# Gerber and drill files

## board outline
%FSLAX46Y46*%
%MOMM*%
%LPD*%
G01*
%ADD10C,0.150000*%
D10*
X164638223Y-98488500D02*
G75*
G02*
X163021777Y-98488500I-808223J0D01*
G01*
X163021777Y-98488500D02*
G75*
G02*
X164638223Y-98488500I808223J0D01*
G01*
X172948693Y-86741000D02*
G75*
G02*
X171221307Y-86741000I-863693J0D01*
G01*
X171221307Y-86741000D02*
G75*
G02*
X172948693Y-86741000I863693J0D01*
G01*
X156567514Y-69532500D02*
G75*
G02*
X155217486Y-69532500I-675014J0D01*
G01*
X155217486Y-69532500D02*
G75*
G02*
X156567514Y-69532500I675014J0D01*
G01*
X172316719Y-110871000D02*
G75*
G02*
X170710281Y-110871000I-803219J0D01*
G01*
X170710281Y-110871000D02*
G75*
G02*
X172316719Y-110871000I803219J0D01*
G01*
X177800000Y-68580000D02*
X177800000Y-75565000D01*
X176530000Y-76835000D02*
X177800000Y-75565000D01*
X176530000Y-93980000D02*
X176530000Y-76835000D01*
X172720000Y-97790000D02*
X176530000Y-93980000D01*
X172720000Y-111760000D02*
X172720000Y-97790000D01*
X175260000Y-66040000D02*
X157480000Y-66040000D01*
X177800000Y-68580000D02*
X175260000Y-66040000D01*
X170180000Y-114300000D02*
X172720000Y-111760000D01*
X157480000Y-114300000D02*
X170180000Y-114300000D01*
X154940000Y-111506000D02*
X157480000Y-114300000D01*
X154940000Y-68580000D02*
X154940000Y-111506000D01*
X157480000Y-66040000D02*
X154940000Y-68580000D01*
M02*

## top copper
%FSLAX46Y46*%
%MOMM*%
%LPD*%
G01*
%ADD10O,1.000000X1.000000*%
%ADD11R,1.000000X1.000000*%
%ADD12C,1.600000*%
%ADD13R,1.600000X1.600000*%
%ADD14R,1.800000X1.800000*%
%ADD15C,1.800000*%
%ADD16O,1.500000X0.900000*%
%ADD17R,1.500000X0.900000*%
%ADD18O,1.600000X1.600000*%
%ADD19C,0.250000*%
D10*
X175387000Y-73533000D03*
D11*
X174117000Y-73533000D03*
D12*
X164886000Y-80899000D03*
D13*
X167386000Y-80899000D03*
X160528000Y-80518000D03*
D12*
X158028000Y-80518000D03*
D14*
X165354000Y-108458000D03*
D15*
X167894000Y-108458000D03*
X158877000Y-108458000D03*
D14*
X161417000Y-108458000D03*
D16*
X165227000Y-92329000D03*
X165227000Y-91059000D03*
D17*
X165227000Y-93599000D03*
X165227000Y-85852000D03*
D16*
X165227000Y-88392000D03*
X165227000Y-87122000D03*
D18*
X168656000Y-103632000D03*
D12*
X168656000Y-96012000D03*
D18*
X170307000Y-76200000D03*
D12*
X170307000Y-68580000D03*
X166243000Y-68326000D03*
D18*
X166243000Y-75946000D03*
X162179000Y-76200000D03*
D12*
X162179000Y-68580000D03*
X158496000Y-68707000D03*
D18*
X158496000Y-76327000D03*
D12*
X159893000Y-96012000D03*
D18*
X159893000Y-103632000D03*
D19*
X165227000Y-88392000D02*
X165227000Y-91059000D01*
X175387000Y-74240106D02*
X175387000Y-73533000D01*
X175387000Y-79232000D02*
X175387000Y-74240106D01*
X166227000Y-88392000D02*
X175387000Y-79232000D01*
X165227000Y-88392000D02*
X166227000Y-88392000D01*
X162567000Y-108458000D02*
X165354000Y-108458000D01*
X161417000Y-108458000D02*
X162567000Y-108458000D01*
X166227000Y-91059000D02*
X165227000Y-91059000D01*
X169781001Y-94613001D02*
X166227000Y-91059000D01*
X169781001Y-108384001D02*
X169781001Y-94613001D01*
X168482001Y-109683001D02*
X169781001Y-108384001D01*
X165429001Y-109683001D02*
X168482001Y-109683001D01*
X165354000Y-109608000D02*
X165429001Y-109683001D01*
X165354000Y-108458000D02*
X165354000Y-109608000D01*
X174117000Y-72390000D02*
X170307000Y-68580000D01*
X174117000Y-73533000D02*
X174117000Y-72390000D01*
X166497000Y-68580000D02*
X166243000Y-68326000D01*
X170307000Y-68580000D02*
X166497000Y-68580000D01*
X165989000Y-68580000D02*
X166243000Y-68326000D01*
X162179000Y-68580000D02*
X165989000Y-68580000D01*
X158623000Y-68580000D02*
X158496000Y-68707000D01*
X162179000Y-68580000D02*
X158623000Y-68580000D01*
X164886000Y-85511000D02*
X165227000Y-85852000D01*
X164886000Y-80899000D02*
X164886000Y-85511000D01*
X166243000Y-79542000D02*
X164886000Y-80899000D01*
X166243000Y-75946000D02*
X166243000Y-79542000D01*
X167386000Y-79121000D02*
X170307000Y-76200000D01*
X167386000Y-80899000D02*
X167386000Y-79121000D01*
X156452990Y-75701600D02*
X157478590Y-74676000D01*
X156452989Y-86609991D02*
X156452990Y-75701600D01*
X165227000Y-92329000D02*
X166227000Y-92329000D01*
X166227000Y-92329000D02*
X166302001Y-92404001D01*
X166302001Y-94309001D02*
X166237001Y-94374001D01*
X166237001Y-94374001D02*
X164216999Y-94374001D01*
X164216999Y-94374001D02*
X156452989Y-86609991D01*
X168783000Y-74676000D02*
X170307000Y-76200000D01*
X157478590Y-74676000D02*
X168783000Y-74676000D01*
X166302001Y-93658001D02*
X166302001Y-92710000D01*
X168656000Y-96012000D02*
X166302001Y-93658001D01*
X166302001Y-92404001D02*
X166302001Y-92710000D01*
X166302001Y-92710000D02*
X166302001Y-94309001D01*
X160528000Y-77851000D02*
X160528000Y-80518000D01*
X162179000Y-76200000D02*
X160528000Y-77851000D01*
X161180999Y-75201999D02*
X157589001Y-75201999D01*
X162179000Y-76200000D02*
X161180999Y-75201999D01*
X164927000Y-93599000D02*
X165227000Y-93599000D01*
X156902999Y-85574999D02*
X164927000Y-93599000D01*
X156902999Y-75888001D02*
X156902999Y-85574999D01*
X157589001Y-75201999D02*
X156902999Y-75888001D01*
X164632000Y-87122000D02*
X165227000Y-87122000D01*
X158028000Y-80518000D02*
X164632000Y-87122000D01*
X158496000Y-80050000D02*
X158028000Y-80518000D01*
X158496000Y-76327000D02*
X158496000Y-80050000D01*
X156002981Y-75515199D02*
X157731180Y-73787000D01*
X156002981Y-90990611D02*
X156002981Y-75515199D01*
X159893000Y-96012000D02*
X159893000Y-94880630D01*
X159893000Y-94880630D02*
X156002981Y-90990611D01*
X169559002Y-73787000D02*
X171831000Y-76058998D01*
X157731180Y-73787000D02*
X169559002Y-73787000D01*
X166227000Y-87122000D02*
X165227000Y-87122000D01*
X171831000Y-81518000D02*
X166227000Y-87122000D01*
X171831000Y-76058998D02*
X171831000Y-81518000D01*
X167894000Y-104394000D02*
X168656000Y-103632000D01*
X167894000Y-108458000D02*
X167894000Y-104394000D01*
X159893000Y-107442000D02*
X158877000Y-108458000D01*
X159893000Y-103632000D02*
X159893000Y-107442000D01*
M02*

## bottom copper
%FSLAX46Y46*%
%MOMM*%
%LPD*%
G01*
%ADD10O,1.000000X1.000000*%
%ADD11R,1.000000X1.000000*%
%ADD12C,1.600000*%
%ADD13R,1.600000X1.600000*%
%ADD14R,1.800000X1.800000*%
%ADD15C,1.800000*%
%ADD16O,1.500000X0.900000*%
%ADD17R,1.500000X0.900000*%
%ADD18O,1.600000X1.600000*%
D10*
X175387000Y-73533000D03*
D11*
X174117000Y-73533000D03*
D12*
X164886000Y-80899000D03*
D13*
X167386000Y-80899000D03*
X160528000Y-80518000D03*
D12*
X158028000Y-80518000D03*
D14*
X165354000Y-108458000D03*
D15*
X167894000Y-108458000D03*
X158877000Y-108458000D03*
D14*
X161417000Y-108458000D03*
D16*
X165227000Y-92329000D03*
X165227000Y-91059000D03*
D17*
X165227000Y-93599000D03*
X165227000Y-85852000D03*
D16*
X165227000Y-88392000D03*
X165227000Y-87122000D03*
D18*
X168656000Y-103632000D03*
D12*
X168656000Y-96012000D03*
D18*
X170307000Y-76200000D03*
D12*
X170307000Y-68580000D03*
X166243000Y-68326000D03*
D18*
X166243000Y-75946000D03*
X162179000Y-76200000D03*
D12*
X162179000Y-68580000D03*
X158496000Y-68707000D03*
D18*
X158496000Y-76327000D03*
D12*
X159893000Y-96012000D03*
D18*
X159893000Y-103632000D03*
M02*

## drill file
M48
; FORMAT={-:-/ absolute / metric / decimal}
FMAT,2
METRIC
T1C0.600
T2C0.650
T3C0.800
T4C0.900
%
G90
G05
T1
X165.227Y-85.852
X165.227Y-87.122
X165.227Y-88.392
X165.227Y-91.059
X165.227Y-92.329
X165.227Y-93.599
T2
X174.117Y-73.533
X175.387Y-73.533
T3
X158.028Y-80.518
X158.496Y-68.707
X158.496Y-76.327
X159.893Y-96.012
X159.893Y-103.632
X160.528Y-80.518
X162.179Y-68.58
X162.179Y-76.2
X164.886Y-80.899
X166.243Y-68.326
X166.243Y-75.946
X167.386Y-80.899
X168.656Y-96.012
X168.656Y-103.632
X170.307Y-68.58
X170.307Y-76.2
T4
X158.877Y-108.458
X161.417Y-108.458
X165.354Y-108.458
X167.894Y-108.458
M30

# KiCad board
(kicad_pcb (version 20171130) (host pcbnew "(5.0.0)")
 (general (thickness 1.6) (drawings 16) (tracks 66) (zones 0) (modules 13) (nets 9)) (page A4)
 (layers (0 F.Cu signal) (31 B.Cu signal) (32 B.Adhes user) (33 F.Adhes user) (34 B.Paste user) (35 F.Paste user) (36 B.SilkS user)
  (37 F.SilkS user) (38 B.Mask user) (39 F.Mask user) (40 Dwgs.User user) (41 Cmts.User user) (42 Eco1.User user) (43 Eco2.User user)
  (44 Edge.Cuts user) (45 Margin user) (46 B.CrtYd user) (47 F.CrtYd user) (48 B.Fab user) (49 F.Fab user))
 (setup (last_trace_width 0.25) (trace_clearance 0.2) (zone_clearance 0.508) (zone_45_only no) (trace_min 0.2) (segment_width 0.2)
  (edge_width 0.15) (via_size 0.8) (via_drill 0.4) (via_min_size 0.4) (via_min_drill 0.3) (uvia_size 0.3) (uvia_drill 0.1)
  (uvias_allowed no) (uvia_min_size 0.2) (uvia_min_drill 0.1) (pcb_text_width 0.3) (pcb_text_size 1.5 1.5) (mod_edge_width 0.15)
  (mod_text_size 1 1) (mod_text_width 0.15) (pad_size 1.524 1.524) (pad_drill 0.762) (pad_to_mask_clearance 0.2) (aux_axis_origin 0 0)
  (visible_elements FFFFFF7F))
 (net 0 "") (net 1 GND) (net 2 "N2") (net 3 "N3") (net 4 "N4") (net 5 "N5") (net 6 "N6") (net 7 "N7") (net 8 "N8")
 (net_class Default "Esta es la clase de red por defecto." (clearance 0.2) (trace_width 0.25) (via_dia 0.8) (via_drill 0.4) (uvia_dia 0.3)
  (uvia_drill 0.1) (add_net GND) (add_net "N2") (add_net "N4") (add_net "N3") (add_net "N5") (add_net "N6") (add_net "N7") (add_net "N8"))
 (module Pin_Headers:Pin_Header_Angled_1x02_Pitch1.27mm (layer F.Cu) (at 174.117 73.533 90)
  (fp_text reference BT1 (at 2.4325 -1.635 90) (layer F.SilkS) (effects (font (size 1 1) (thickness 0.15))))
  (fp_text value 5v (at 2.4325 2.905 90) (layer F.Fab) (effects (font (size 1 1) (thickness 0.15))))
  (pad 2 thru_hole oval (at 0 1.27 90) (size 1 1) (drill 0.65) (layers *.Cu *.Mask) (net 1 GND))
  (pad 1 thru_hole rect (at 0 0 90) (size 1 1) (drill 0.65) (layers *.Cu *.Mask) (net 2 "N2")))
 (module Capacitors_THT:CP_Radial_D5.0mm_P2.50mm (layer F.Cu) (at 167.386 80.899 180)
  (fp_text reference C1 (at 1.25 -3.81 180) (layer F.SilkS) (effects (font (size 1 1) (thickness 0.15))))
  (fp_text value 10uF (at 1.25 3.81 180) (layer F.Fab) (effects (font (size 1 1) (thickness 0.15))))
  (pad 2 thru_hole circle (at 2.5 0 180) (size 1.6 1.6) (drill 0.8) (layers *.Cu *.Mask) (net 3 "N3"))
  (pad 1 thru_hole rect (at 0 0 180) (size 1.6 1.6) (drill 0.8) (layers *.Cu *.Mask) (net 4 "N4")))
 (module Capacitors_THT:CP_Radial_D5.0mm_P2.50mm (layer F.Cu) (at 160.528 80.518 180)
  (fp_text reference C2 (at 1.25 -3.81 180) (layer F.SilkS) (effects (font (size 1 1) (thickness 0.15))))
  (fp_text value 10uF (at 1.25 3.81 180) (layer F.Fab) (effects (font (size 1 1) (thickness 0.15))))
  (pad 1 thru_hole rect (at 0 0 180) (size 1.6 1.6) (drill 0.8) (layers *.Cu *.Mask) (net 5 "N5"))
  (pad 2 thru_hole circle (at 2.5 0 180) (size 1.6 1.6) (drill 0.8) (layers *.Cu *.Mask) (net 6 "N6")))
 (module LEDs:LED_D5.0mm (layer F.Cu) (at 165.354 108.458)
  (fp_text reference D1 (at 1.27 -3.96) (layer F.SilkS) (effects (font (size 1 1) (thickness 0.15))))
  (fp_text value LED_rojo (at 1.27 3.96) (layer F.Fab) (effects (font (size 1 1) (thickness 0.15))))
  (pad 1 thru_hole rect (at 0 0) (size 1.8 1.8) (drill 0.9) (layers *.Cu *.Mask) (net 1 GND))
  (pad 2 thru_hole circle (at 2.54 0) (size 1.8 1.8) (drill 0.9) (layers *.Cu *.Mask) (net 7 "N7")))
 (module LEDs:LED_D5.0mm (layer F.Cu) (at 161.417 108.458 180)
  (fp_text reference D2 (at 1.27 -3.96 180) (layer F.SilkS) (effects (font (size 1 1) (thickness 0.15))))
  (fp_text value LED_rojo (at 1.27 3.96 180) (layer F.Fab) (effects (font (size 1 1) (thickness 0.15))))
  (pad 2 thru_hole circle (at 2.54 0 180) (size 1.8 1.8) (drill 0.9) (layers *.Cu *.Mask) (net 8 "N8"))
  (pad 1 thru_hole rect (at 0 0 180) (size 1.8 1.8) (drill 0.9) (layers *.Cu *.Mask) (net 1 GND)))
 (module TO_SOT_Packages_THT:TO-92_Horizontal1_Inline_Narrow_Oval (layer F.Cu) (at 165.227 93.599 90)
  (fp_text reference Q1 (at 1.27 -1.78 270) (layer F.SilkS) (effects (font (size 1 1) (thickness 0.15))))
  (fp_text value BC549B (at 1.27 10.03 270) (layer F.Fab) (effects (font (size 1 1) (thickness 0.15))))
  (pad 2 thru_hole oval (at 1.27 0 270) (size 0.9 1.5) (drill 0.6) (layers *.Cu *.Mask) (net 4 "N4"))
  (pad 3 thru_hole oval (at 2.54 0 270) (size 0.9 1.5) (drill 0.6) (layers *.Cu *.Mask) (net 1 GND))
  (pad 1 thru_hole rect (at 0 0 270) (size 0.9 1.5) (drill 0.6) (layers *.Cu *.Mask) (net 5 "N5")))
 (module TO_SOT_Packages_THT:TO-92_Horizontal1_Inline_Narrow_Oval (layer F.Cu) (at 165.227 85.852 270)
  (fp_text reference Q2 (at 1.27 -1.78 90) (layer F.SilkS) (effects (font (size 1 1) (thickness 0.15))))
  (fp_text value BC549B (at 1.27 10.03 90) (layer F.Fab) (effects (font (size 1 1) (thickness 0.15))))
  (pad 1 thru_hole rect (at 0 0 90) (size 0.9 1.5) (drill 0.6) (layers *.Cu *.Mask) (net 3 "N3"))
  (pad 3 thru_hole oval (at 2.54 0 90) (size 0.9 1.5) (drill 0.6) (layers *.Cu *.Mask) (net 1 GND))
  (pad 2 thru_hole oval (at 1.27 0 90) (size 0.9 1.5) (drill 0.6) (layers *.Cu *.Mask) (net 6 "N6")))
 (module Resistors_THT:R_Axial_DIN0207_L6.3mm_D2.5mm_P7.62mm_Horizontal (layer F.Cu) (at 168.656 96.012 270)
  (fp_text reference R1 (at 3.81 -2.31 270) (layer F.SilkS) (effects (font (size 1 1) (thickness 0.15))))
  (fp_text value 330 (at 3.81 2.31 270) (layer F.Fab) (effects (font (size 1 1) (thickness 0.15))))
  (pad 2 thru_hole oval (at 7.62 0 270) (size 1.6 1.6) (drill 0.8) (layers *.Cu *.Mask) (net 7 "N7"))
  (pad 1 thru_hole circle (at 0 0 270) (size 1.6 1.6) (drill 0.8) (layers *.Cu *.Mask) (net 4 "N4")))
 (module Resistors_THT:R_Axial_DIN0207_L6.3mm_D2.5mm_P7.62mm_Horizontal (layer F.Cu) (at 170.307 68.58 270)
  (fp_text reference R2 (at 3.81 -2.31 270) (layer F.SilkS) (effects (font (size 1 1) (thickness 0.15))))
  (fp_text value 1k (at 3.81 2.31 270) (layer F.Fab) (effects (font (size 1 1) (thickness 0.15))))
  (pad 2 thru_hole oval (at 7.62 0 270) (size 1.6 1.6) (drill 0.8) (layers *.Cu *.Mask) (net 4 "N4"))
  (pad 1 thru_hole circle (at 0 0 270) (size 1.6 1.6) (drill 0.8) (layers *.Cu *.Mask) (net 2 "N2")))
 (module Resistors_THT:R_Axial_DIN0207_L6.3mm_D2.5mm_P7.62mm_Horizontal (layer F.Cu) (at 166.243 68.326 270)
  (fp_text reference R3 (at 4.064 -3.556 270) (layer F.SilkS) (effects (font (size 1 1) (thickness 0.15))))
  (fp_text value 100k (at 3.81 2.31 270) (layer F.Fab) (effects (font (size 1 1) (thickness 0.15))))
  (pad 1 thru_hole circle (at 0 0 270) (size 1.6 1.6) (drill 0.8) (layers *.Cu *.Mask) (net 2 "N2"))
  (pad 2 thru_hole oval (at 7.62 0 270) (size 1.6 1.6) (drill 0.8) (layers *.Cu *.Mask) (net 3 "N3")))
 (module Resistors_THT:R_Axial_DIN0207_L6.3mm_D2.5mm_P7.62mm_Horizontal (layer F.Cu) (at 162.179 68.58 270)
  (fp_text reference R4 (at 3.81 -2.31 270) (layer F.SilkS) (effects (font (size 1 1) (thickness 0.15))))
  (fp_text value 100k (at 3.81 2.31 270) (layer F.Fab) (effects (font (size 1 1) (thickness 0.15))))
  (pad 2 thru_hole oval (at 7.62 0 270) (size 1.6 1.6) (drill 0.8) (layers *.Cu *.Mask) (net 5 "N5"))
  (pad 1 thru_hole circle (at 0 0 270) (size 1.6 1.6) (drill 0.8) (layers *.Cu *.Mask) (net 2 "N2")))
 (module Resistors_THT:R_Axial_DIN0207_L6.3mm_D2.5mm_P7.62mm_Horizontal (layer F.Cu) (at 158.496 68.707 270)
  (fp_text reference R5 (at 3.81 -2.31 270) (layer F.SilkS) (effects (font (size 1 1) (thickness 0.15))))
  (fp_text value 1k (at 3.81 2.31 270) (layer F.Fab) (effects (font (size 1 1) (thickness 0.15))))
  (pad 1 thru_hole circle (at 0 0 270) (size 1.6 1.6) (drill 0.8) (layers *.Cu *.Mask) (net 2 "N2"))
  (pad 2 thru_hole oval (at 7.62 0 270) (size 1.6 1.6) (drill 0.8) (layers *.Cu *.Mask) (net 6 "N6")))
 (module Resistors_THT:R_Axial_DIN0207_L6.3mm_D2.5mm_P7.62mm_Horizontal (layer F.Cu) (at 159.893 96.012 270)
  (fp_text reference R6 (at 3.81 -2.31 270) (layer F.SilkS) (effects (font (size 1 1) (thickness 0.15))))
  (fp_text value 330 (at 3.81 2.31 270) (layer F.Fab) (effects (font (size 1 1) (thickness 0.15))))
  (pad 1 thru_hole circle (at 0 0 270) (size 1.6 1.6) (drill 0.8) (layers *.Cu *.Mask) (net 6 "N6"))
  (pad 2 thru_hole oval (at 7.62 0 270) (size 1.6 1.6) (drill 0.8) (layers *.Cu *.Mask) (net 8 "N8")))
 (gr_circle (center 163.83 98.4885) (end 164.4015 97.917) (layer Edge.Cuts) (width 0.15))
 (gr_circle (center 172.085 86.741) (end 172.593 86.0425) (layer Edge.Cuts) (width 0.15))
 (gr_circle (center 155.8925 69.5325) (end 156.337 69.0245) (layer Edge.Cuts) (width 0.15))
 (gr_circle (center 171.5135 110.871) (end 171.7675 111.633) (layer Edge.Cuts) (width 0.15))
 (gr_line (start 177.8 68.58) (end 177.8 75.565) (layer Edge.Cuts) (width 0.15))
 (gr_line (start 176.53 76.835) (end 177.8 75.565) (layer Edge.Cuts) (width 0.15))
 (gr_line (start 176.53 93.98) (end 176.53 76.835) (layer Edge.Cuts) (width 0.15))
 (gr_line (start 172.72 97.79) (end 176.53 93.98) (layer Edge.Cuts) (width 0.15))
 (gr_line (start 172.72 111.76) (end 172.72 97.79) (layer Edge.Cuts) (width 0.15))
 (gr_line (start 175.26 66.04) (end 157.48 66.04) (layer Edge.Cuts) (width 0.15))
 (gr_line (start 177.8 68.58) (end 175.26 66.04) (layer Edge.Cuts) (width 0.15))
 (gr_line (start 170.18 114.3) (end 172.72 111.76) (layer Edge.Cuts) (width 0.15))
 (gr_line (start 157.48 114.3) (end 170.18 114.3) (layer Edge.Cuts) (width 0.15))
 (gr_line (start 154.94 111.506) (end 157.48 114.3) (layer Edge.Cuts) (width 0.15))
 (gr_line (start 154.94 68.58) (end 154.94 111.506) (layer Edge.Cuts) (width 0.15))
 (gr_line (start 157.48 66.04) (end 154.94 68.58) (layer Edge.Cuts) (width 0.15))
 (segment (start 165.227 88.392) (end 165.227 91.059) (width 0.25) (layer F.Cu) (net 1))
 (segment (start 175.387 74.240106) (end 175.387 73.533) (width 0.25) (layer F.Cu) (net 1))
 (segment (start 175.387 79.232) (end 175.387 74.240106) (width 0.25) (layer F.Cu) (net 1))
 (segment (start 166.227 88.392) (end 175.387 79.232) (width 0.25) (layer F.Cu) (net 1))
 (segment (start 165.227 88.392) (end 166.227 88.392) (width 0.25) (layer F.Cu) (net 1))
 (segment (start 162.567 108.458) (end 165.354 108.458) (width 0.25) (layer F.Cu) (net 1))
 (segment (start 161.417 108.458) (end 162.567 108.458) (width 0.25) (layer F.Cu) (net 1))
 (segment (start 166.227 91.059) (end 165.227 91.059) (width 0.25) (layer F.Cu) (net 1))
 (segment (start 169.781001 94.613001) (end 166.227 91.059) (width 0.25) (layer F.Cu) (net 1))
 (segment (start 169.781001 108.384001) (end 169.781001 94.613001) (width 0.25) (layer F.Cu) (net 1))
 (segment (start 168.482001 109.683001) (end 169.781001 108.384001) (width 0.25) (layer F.Cu) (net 1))
 (segment (start 165.429001 109.683001) (end 168.482001 109.683001) (width 0.25) (layer F.Cu) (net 1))
 (segment (start 165.354 109.608) (end 165.429001 109.683001) (width 0.25) (layer F.Cu) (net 1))
 (segment (start 165.354 108.458) (end 165.354 109.608) (width 0.25) (layer F.Cu) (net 1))
 (segment (start 174.117 72.39) (end 170.307 68.58) (width 0.25) (layer F.Cu) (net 2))
 (segment (start 174.117 73.533) (end 174.117 72.39) (width 0.25) (layer F.Cu) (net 2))
 (segment (start 166.497 68.58) (end 166.243 68.326) (width 0.25) (layer F.Cu) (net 2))
 (segment (start 170.307 68.58) (end 166.497 68.58) (width 0.25) (layer F.Cu) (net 2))
 (segment (start 165.989 68.58) (end 166.243 68.326) (width 0.25) (layer F.Cu) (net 2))
 (segment (start 162.179 68.58) (end 165.989 68.58) (width 0.25) (layer F.Cu) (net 2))
 (segment (start 158.623 68.58) (end 158.496 68.707) (width 0.25) (layer F.Cu) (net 2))
 (segment (start 162.179 68.58) (end 158.623 68.58) (width 0.25) (layer F.Cu) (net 2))
 (segment (start 164.886 85.511) (end 165.227 85.852) (width 0.25) (layer F.Cu) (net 3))
 (segment (start 164.886 80.899) (end 164.886 85.511) (width 0.25) (layer F.Cu) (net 3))
 (segment (start 166.243 79.542) (end 164.886 80.899) (width 0.25) (layer F.Cu) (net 3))
 (segment (start 166.243 75.946) (end 166.243 79.542) (width 0.25) (layer F.Cu) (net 3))
 (segment (start 167.386 79.121) (end 170.307 76.2) (width 0.25) (layer F.Cu) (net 4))
 (segment (start 167.386 80.899) (end 167.386 79.121) (width 0.25) (layer F.Cu) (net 4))
 (segment (start 156.45299 75.7016) (end 157.47859 74.676) (width 0.25) (layer F.Cu) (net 4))
 (segment (start 156.452989 86.609991) (end 156.45299 75.7016) (width 0.25) (layer F.Cu) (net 4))
 (segment (start 165.227 92.329) (end 166.227 92.329) (width 0.25) (layer F.Cu) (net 4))
 (segment (start 166.227 92.329) (end 166.302001 92.404001) (width 0.25) (layer F.Cu) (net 4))
 (segment (start 166.302001 94.309001) (end 166.237001 94.374001) (width 0.25) (layer F.Cu) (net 4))
 (segment (start 166.237001 94.374001) (end 164.216999 94.374001) (width 0.25) (layer F.Cu) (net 4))
 (segment (start 164.216999 94.374001) (end 156.452989 86.609991) (width 0.25) (layer F.Cu) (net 4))
 (segment (start 168.783 74.676) (end 170.307 76.2) (width 0.25) (layer F.Cu) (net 4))
 (segment (start 157.47859 74.676) (end 168.783 74.676) (width 0.25) (layer F.Cu) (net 4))
 (segment (start 166.302001 93.658001) (end 166.302001 92.71) (width 0.25) (layer F.Cu) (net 4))
 (segment (start 168.656 96.012) (end 166.302001 93.658001) (width 0.25) (layer F.Cu) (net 4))
 (segment (start 166.302001 92.404001) (end 166.302001 92.71) (width 0.25) (layer F.Cu) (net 4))
 (segment (start 166.302001 92.71) (end 166.302001 94.309001) (width 0.25) (layer F.Cu) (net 4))
 (segment (start 160.528 77.851) (end 160.528 80.518) (width 0.25) (layer F.Cu) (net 5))
 (segment (start 162.179 76.2) (end 160.528 77.851) (width 0.25) (layer F.Cu) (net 5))
 (segment (start 161.180999 75.201999) (end 157.589001 75.201999) (width 0.25) (layer F.Cu) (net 5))
 (segment (start 162.179 76.2) (end 161.180999 75.201999) (width 0.25) (layer F.Cu) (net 5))
 (segment (start 164.927 93.599) (end 165.227 93.599) (width 0.25) (layer F.Cu) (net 5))
 (segment (start 156.902999 85.574999) (end 164.927 93.599) (width 0.25) (layer F.Cu) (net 5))
 (segment (start 156.902999 75.888001) (end 156.902999 85.574999) (width 0.25) (layer F.Cu) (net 5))
 (segment (start 157.589001 75.201999) (end 156.902999 75.888001) (width 0.25) (layer F.Cu) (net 5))
 (segment (start 164.632 87.122) (end 165.227 87.122) (width 0.25) (layer F.Cu) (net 6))
 (segment (start 158.028 80.518) (end 164.632 87.122) (width 0.25) (layer F.Cu) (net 6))
 (segment (start 158.496 80.05) (end 158.028 80.518) (width 0.25) (layer F.Cu) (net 6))
 (segment (start 158.496 76.327) (end 158.496 80.05) (width 0.25) (layer F.Cu) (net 6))
 (segment (start 156.002981 75.515199) (end 157.73118 73.787) (width 0.25) (layer F.Cu) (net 6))
 (segment (start 156.002981 90.990611) (end 156.002981 75.515199) (width 0.25) (layer F.Cu) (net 6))
 (segment (start 159.893 96.012) (end 159.893 94.88063) (width 0.25) (layer F.Cu) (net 6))
 (segment (start 159.893 94.88063) (end 156.002981 90.990611) (width 0.25) (layer F.Cu) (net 6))
 (segment (start 169.559002 73.787) (end 171.831 76.058998) (width 0.25) (layer F.Cu) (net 6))
 (segment (start 157.73118 73.787) (end 169.559002 73.787) (width 0.25) (layer F.Cu) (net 6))
 (segment (start 166.227 87.122) (end 165.227 87.122) (width 0.25) (layer F.Cu) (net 6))
 (segment (start 171.831 81.518) (end 166.227 87.122) (width 0.25) (layer F.Cu) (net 6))
 (segment (start 171.831 76.058998) (end 171.831 81.518) (width 0.25) (layer F.Cu) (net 6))
 (segment (start 167.894 104.394) (end 168.656 103.632) (width 0.25) (layer F.Cu) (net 7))
 (segment (start 167.894 108.458) (end 167.894 104.394) (width 0.25) (layer F.Cu) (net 7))
 (segment (start 159.893 107.442) (end 158.877 108.458) (width 0.25) (layer F.Cu) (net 8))
 (segment (start 159.893 103.632) (end 159.893 107.442) (width 0.25) (layer F.Cu) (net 8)))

